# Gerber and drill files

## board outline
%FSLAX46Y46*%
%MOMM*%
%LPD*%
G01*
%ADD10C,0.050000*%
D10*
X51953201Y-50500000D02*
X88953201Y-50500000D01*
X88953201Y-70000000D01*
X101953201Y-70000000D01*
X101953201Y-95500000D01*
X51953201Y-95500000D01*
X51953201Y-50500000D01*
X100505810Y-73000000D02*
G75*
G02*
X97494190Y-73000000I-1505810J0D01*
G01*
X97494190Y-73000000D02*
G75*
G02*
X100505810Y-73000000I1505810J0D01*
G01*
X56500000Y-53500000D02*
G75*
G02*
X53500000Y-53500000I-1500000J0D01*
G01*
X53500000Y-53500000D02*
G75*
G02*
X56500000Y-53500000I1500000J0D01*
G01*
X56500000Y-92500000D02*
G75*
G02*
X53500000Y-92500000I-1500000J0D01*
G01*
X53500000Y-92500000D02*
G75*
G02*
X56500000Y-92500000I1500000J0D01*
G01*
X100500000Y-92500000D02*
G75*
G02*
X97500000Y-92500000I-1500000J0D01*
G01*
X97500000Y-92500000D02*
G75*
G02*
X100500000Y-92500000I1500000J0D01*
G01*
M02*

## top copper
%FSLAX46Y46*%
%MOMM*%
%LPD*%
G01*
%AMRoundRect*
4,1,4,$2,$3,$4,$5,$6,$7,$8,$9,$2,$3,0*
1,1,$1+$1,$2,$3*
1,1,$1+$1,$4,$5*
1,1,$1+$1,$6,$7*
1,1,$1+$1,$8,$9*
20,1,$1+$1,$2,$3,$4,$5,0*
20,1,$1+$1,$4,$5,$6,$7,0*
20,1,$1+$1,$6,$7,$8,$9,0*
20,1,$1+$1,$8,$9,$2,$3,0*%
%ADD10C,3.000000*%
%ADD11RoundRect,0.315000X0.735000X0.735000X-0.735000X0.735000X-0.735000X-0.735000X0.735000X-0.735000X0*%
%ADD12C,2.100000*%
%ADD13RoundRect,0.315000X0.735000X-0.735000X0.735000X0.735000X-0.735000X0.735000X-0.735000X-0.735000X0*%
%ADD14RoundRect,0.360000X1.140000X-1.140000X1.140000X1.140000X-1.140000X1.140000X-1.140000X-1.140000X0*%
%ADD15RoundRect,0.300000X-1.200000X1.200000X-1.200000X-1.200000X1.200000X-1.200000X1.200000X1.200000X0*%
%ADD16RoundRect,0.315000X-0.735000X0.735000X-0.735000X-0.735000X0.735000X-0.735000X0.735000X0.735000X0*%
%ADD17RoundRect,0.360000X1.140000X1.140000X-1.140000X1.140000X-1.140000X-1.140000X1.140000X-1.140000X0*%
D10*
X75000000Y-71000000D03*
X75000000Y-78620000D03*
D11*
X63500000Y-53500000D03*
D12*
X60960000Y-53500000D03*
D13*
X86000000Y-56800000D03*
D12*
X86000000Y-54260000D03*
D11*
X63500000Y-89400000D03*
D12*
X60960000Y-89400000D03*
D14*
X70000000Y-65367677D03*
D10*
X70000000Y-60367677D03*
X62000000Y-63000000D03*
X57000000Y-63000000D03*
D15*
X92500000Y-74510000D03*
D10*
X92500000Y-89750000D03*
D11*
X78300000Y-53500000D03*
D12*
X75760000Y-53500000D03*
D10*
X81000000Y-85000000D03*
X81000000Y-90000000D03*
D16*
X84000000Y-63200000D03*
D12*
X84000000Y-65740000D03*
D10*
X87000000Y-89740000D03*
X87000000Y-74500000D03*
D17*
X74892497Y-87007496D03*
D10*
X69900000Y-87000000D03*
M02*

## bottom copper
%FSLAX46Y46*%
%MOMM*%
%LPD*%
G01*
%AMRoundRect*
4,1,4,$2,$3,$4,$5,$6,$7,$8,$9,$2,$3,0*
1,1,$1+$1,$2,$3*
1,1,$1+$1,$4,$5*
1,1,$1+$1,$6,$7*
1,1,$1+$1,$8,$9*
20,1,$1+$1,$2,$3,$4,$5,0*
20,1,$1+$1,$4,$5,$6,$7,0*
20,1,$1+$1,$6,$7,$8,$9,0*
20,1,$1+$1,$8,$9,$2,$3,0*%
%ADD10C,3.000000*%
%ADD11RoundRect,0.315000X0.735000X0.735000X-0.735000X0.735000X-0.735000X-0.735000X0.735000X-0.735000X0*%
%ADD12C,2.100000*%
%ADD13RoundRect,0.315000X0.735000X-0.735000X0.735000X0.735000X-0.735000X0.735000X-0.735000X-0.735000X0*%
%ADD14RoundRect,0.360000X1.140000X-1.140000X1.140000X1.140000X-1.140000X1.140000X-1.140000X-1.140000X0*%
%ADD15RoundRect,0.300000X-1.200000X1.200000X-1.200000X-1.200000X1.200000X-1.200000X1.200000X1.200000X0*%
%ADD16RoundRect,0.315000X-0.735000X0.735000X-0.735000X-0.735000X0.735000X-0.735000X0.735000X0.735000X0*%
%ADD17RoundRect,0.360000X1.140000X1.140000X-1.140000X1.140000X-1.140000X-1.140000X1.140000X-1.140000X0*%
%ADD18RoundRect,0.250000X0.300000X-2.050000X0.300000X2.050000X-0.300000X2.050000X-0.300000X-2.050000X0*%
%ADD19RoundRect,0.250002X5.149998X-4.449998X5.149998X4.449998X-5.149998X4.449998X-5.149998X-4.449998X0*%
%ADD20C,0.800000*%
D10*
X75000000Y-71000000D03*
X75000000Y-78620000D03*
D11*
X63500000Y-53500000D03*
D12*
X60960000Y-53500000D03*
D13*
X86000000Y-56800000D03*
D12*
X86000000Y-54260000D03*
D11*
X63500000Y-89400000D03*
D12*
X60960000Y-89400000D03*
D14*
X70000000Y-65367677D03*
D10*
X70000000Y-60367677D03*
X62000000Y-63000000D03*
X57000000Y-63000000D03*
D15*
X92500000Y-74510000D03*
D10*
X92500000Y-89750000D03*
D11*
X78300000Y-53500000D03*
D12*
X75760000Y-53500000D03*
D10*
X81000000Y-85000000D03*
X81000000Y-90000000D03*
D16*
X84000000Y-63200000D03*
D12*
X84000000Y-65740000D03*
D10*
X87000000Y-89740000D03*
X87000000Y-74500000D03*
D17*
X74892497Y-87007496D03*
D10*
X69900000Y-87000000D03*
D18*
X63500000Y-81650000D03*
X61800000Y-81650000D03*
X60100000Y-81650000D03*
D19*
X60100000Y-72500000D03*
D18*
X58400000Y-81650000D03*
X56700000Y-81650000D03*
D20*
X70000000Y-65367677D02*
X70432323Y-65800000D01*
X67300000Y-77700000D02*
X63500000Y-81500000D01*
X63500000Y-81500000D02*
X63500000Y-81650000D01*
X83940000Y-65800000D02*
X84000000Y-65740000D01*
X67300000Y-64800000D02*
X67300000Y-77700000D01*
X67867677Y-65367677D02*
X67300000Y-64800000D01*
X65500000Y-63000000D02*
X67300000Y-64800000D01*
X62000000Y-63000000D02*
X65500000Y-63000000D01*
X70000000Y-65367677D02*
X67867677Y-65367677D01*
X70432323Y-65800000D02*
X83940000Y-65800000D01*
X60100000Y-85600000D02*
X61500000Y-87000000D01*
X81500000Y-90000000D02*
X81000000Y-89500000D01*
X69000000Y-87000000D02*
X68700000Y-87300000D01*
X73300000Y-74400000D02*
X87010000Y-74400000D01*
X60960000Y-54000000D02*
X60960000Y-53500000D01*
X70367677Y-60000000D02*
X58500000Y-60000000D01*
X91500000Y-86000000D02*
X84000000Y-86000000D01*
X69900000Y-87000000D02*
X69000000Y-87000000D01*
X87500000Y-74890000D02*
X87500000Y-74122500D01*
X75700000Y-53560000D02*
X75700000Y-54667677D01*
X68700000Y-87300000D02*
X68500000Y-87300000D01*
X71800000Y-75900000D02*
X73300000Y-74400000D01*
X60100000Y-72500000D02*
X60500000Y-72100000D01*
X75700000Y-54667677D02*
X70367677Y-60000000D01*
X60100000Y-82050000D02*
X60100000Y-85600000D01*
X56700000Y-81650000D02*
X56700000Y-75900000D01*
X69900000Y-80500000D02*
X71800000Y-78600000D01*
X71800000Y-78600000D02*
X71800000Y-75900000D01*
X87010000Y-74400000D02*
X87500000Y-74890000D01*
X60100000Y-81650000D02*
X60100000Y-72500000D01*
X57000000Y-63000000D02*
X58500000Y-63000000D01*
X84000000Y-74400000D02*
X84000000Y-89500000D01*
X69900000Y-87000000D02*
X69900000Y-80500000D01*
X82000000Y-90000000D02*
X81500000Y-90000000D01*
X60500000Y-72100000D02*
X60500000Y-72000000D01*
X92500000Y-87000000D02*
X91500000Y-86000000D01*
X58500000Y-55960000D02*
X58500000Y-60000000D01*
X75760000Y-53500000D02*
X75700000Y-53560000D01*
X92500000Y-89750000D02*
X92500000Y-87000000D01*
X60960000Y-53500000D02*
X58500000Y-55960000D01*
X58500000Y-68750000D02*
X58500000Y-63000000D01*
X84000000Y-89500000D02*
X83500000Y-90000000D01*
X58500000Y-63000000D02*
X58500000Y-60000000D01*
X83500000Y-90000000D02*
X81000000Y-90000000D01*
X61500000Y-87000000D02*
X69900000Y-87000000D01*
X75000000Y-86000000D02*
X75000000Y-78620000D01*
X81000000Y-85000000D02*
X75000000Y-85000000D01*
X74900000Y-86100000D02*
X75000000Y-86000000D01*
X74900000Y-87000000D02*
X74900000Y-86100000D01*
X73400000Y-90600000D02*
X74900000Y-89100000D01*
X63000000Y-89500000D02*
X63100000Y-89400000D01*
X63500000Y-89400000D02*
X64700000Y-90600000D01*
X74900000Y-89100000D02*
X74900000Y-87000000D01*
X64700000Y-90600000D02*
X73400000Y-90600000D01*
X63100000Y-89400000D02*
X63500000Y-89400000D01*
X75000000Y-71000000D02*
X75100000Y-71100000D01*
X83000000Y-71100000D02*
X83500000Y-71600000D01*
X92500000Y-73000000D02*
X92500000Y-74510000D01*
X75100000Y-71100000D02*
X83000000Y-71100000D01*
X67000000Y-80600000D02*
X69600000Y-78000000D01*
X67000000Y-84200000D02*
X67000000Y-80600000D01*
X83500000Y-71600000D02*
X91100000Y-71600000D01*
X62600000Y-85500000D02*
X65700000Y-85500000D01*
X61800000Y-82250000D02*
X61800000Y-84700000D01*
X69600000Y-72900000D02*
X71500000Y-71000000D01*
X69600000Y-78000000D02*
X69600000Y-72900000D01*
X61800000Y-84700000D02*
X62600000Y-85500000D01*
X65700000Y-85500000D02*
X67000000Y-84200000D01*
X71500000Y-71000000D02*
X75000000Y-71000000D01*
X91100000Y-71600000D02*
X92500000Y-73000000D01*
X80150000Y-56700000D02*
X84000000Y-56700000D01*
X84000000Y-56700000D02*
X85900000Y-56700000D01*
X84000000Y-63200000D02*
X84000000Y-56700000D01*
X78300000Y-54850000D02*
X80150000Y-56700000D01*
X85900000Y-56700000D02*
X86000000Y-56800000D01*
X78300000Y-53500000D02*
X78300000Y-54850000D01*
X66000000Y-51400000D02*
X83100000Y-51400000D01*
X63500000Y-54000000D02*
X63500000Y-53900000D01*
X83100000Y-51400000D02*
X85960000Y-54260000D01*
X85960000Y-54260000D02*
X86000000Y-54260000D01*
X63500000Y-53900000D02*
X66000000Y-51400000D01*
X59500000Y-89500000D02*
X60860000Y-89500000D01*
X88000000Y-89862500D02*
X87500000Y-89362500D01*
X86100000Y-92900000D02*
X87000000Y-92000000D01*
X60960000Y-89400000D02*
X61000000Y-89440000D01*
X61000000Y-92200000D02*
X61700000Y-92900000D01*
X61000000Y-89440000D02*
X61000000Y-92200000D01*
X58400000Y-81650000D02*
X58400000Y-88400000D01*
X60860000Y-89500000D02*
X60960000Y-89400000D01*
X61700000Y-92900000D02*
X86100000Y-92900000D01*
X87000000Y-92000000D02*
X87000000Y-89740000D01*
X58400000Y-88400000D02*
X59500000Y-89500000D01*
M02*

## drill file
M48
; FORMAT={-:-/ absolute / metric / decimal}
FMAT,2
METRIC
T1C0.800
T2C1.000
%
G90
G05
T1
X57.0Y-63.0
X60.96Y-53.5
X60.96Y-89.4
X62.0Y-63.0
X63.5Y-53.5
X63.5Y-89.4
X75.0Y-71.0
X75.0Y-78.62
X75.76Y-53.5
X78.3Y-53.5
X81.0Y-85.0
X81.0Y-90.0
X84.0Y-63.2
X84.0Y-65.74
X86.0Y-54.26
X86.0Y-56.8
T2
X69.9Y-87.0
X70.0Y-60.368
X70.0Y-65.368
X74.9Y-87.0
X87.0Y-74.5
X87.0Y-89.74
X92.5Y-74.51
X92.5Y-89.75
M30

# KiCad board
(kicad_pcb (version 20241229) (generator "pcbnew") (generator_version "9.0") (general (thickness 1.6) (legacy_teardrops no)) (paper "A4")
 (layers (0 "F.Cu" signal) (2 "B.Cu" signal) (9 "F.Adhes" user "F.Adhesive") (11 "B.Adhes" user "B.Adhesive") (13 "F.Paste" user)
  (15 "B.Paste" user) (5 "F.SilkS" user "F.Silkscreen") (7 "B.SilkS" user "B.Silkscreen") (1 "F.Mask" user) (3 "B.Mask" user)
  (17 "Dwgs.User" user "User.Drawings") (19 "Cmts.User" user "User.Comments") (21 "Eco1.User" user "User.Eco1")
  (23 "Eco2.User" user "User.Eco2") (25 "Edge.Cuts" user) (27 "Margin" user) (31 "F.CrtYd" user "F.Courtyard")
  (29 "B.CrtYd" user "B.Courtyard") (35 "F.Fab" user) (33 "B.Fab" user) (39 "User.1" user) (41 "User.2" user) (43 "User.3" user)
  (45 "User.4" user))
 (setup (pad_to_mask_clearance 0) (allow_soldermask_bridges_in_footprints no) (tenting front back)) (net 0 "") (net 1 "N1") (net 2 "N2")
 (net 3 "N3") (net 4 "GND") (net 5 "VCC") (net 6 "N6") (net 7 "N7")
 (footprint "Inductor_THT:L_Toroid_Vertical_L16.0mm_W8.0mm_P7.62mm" (layer "F.Cu") (at 75 71)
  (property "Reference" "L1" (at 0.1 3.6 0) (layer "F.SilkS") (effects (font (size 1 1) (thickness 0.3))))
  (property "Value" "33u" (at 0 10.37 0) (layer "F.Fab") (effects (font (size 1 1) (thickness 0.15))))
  (pad "1" thru_hole circle (at 0 0) (size 3 3) (drill 0.8) (layers "*.Cu" "*.Mask") (remove_unused_layers no) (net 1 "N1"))
  (pad "2" thru_hole circle (at 0 7.62) (size 3 3) (drill 0.8) (layers "*.Cu" "*.Mask") (remove_unused_layers no) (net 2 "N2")))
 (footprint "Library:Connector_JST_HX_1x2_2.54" (layer "F.Cu") (at 63.5 53.5 180)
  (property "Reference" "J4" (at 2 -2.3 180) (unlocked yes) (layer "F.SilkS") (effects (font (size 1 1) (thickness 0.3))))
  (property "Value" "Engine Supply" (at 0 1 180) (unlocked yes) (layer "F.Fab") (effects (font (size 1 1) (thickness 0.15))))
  (pad "1" thru_hole roundrect (at 0 0 180) (size 2.1 2.1) (drill 0.8) (layers "*.Cu" "*.Mask") (remove_unused_layers no)
   (roundrect_rratio 0.15) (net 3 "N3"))
  (pad "2" thru_hole circle (at 2.54 0 180) (size 2.1 2.1) (drill 0.8) (layers "*.Cu" "*.Mask") (remove_unused_layers no) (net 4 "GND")))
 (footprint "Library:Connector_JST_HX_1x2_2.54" (layer "F.Cu") (at 86 56.8 90)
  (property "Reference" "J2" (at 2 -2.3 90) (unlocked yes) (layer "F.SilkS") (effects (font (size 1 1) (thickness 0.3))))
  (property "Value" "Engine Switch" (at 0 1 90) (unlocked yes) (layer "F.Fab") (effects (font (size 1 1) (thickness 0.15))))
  (pad "1" thru_hole roundrect (at 0 0 90) (size 2.1 2.1) (drill 0.8) (layers "*.Cu" "*.Mask") (remove_unused_layers no)
   (roundrect_rratio 0.15) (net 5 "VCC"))
  (pad "2" thru_hole circle (at 2.54 0 90) (size 2.1 2.1) (drill 0.8) (layers "*.Cu" "*.Mask") (remove_unused_layers no) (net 3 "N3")))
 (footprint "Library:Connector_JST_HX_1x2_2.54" (layer "F.Cu") (at 63.5 89.4 180)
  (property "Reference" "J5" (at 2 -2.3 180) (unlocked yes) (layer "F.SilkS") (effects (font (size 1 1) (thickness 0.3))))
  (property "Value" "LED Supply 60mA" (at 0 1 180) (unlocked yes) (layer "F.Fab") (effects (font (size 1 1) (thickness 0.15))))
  (pad "1" thru_hole roundrect (at 0 0 180) (size 2.1 2.1) (drill 0.8) (layers "*.Cu" "*.Mask") (remove_unused_layers no)
   (roundrect_rratio 0.15) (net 2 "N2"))
  (pad "2" thru_hole circle (at 2.54 0 180) (size 2.1 2.1) (drill 0.8) (layers "*.Cu" "*.Mask") (remove_unused_layers no) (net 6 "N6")))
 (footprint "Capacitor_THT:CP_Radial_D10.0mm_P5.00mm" (layer "F.Cu") (at 70 65.367677 90)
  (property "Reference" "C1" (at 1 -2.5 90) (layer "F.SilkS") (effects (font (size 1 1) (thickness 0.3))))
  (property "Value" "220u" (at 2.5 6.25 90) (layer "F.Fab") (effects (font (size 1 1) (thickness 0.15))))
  (pad "1" thru_hole roundrect (at 0 0 90) (size 3 3) (drill 1) (layers "*.Cu" "*.Mask") (remove_unused_layers no) (roundrect_rratio 0.12)
   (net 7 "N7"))
  (pad "2" thru_hole circle (at 5 0 90) (size 3 3) (drill 1) (layers "*.Cu" "*.Mask") (remove_unused_layers no) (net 4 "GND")))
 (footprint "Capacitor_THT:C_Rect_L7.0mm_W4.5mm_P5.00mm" (layer "F.Cu") (at 62 63 180)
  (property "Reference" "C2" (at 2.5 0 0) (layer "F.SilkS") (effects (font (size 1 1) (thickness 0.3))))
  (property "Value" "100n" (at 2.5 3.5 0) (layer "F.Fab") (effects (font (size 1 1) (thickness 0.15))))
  (pad "1" thru_hole circle (at 0 0 180) (size 3 3) (drill 0.8) (layers "*.Cu" "*.Mask") (remove_unused_layers no) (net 7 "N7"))
  (pad "2" thru_hole circle (at 5 0 180) (size 3 3) (drill 0.8) (layers "*.Cu" "*.Mask") (remove_unused_layers no) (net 4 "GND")))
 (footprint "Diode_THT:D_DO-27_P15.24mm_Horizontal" (layer "F.Cu") (at 92.5 74.51 -90)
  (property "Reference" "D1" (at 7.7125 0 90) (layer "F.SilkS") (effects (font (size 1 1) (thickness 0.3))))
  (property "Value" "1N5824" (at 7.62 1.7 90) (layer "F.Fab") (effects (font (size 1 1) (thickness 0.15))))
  (pad "1" thru_hole roundrect (at 0 0 270) (size 3 3) (drill 1) (layers "*.Cu" "*.Mask") (remove_unused_layers no) (roundrect_rratio 0.1)
   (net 1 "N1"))
  (pad "2" thru_hole circle (at 15.24 0 270) (size 3 3) (drill 1) (layers "*.Cu" "*.Mask") (remove_unused_layers no) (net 4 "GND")))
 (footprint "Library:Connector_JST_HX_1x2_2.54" (layer "F.Cu") (at 78.3 53.5 180)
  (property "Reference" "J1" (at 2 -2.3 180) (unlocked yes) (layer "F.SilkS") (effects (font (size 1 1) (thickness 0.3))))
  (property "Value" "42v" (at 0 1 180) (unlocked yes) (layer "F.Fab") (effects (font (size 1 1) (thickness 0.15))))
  (pad "1" thru_hole roundrect (at 0 0 180) (size 2.1 2.1) (drill 0.8) (layers "*.Cu" "*.Mask") (remove_unused_layers no)
   (roundrect_rratio 0.15) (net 5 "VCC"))
  (pad "2" thru_hole circle (at 2.54 0 180) (size 2.1 2.1) (drill 0.8) (layers "*.Cu" "*.Mask") (remove_unused_layers no) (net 4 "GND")))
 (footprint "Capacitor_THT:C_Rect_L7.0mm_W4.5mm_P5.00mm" (layer "F.Cu") (at 81 85 -90)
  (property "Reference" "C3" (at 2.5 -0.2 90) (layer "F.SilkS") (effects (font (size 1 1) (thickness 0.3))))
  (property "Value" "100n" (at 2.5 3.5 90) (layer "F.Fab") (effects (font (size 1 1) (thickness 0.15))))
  (pad "1" thru_hole circle (at 0 0 270) (size 3 3) (drill 0.8) (layers "*.Cu" "*.Mask") (remove_unused_layers no) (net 2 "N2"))
  (pad "2" thru_hole circle (at 5 0 270) (size 3 3) (drill 0.8) (layers "*.Cu" "*.Mask") (remove_unused_layers no) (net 4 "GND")))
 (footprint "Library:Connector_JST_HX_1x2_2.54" (layer "F.Cu") (at 84 63.2 -90)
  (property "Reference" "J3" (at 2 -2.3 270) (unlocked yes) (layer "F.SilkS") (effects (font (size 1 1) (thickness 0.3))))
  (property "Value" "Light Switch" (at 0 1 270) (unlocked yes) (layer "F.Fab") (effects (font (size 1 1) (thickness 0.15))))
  (pad "1" thru_hole roundrect (at 0 0 270) (size 2.1 2.1) (drill 0.8) (layers "*.Cu" "*.Mask") (remove_unused_layers no)
   (roundrect_rratio 0.15) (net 5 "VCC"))
  (pad "2" thru_hole circle (at 2.54 0 270) (size 2.1 2.1) (drill 0.8) (layers "*.Cu" "*.Mask") (remove_unused_layers no) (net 7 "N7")))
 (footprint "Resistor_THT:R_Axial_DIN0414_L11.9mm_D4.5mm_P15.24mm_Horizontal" (layer "F.Cu") (at 87 89.74 90)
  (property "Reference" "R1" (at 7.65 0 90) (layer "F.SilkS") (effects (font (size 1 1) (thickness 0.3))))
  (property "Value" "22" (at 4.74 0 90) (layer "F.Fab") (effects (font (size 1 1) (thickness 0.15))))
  (pad "1" thru_hole circle (at 0 0 90) (size 3 3) (drill 1) (layers "*.Cu" "*.Mask") (remove_unused_layers no) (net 6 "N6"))
  (pad "2" thru_hole circle (at 15.24 0 90) (size 3 3) (drill 1) (layers "*.Cu" "*.Mask") (remove_unused_layers no) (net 4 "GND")))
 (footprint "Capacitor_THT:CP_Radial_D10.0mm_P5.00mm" (layer "F.Cu") (at 74.9 87 180)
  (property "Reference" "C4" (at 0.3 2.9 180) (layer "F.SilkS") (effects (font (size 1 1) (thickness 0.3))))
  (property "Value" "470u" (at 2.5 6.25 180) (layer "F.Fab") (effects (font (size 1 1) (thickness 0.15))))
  (pad "1" thru_hole roundrect (at 0 0 180) (size 3 3) (drill 1 (offset 0.007503 -0.007496)) (layers "*.Cu" "*.Mask")
   (remove_unused_layers no) (roundrect_rratio 0.12) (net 2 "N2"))
  (pad "2" thru_hole circle (at 5 0 180) (size 3 3) (drill 1) (layers "*.Cu" "*.Mask") (remove_unused_layers no) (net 4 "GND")))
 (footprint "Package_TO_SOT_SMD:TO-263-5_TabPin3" (layer "B.Cu") (at 60.1 74 90)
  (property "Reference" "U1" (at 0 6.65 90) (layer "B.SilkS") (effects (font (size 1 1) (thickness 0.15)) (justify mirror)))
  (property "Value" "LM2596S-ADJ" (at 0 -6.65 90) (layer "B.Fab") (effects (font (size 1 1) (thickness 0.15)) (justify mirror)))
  (pad "" smd roundrect (at -0.925 -2.775 90) (size 4.55 5.25) (layers "B.Paste") (roundrect_rratio 0.054945))
  (pad "" smd roundrect (at -0.925 2.775 90) (size 4.55 5.25) (layers "B.Paste") (roundrect_rratio 0.054945))
  (pad "" smd roundrect (at 3.925 -2.775 90) (size 4.55 5.25) (layers "B.Paste") (roundrect_rratio 0.054945))
  (pad "" smd roundrect (at 3.925 2.775 90) (size 4.55 5.25) (layers "B.Paste") (roundrect_rratio 0.054945))
  (pad "1" smd roundrect (at -7.65 3.4 90) (size 4.6 1.1) (layers "B.Cu" "B.Mask" "B.Paste") (roundrect_rratio 0.227273) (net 7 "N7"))
  (pad "2" smd roundrect (at -7.65 1.7 90) (size 4.6 1.1) (layers "B.Cu" "B.Mask" "B.Paste") (roundrect_rratio 0.227273) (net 1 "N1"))
  (pad "3" smd roundrect (at -7.65 0 90) (size 4.6 1.1) (layers "B.Cu" "B.Mask" "B.Paste") (roundrect_rratio 0.227273) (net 4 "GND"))
  (pad "3" smd roundrect (at 1.5 0 90) (size 9.4 10.8) (layers "B.Cu" "B.Mask") (roundrect_rratio 0.026596) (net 4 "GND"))
  (pad "4" smd roundrect (at -7.65 -1.7 90) (size 4.6 1.1) (layers "B.Cu" "B.Mask" "B.Paste") (roundrect_rratio 0.227273) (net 6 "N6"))
  (pad "5" smd roundrect (at -7.65 -3.4 90) (size 4.6 1.1) (layers "B.Cu" "B.Mask" "B.Paste") (roundrect_rratio 0.227273) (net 4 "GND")))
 (gr_poly
  (pts (xy 51.953201 50.5) (xy 88.953201 50.5) (xy 88.953201 70) (xy 101.953201 70) (xy 101.953201 95.5) (xy 51.953201 95.5))
  (stroke (width 0.05) (type solid)) (fill no) (layer "Edge.Cuts"))
 (gr_circle (center 99 73) (end 99 71.49419) (stroke (width 0.05) (type default)) (fill no) (layer "Edge.Cuts"))
 (gr_circle (center 55 53.5) (end 55 52) (stroke (width 0.05) (type default)) (fill no) (layer "Edge.Cuts"))
 (gr_circle (center 55 92.5) (end 55 91) (stroke (width 0.05) (type default)) (fill no) (layer "Edge.Cuts"))
 (gr_circle (center 99 92.5) (end 99 94) (stroke (width 0.05) (type default)) (fill no) (layer "Edge.Cuts"))
 (segment (start 70 65.367677) (end 70.432323 65.8) (width 0.8) (layer "B.Cu") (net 7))
 (segment (start 67.3 77.7) (end 63.5 81.5) (width 0.8) (layer "B.Cu") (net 7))
 (segment (start 63.5 81.5) (end 63.5 81.65) (width 0.8) (layer "B.Cu") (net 7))
 (segment (start 83.94 65.8) (end 84 65.74) (width 0.8) (layer "B.Cu") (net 7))
 (segment (start 67.3 64.8) (end 67.3 77.7) (width 0.8) (layer "B.Cu") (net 7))
 (segment (start 67.867677 65.367677) (end 67.3 64.8) (width 0.8) (layer "B.Cu") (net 7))
 (segment (start 65.5 63) (end 67.3 64.8) (width 0.8) (layer "B.Cu") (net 7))
 (segment (start 62 63) (end 65.5 63) (width 0.8) (layer "B.Cu") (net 7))
 (segment (start 70 65.367677) (end 67.867677 65.367677) (width 0.8) (layer "B.Cu") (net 7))
 (segment (start 70.432323 65.8) (end 83.94 65.8) (width 0.8) (layer "B.Cu") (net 7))
 (segment (start 60.1 85.6) (end 61.5 87) (width 0.8) (layer "B.Cu") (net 4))
 (segment (start 81.5 90) (end 81 89.5) (width 0.8) (layer "B.Cu") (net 4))
 (segment (start 69 87) (end 68.7 87.3) (width 0.8) (layer "B.Cu") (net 4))
 (segment (start 73.3 74.4) (end 87.01 74.4) (width 0.8) (layer "B.Cu") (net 4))
 (segment (start 60.96 54) (end 60.96 53.5) (width 0.8) (layer "B.Cu") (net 4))
 (segment (start 70.367677 60) (end 58.5 60) (width 0.8) (layer "B.Cu") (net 4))
 (segment (start 91.5 86) (end 84 86) (width 0.8) (layer "B.Cu") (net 4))
 (segment (start 69.9 87) (end 69 87) (width 0.8) (layer "B.Cu") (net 4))
 (segment (start 87.5 74.89) (end 87.5 74.1225) (width 0.8) (layer "B.Cu") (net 4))
 (segment (start 75.7 53.56) (end 75.7 54.667677) (width 0.8) (layer "B.Cu") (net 4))
 (segment (start 68.7 87.3) (end 68.5 87.3) (width 0.8) (layer "B.Cu") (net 4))
 (segment (start 71.8 75.9) (end 73.3 74.4) (width 0.8) (layer "B.Cu") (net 4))
 (segment (start 60.1 72.5) (end 60.5 72.1) (width 0.8) (layer "B.Cu") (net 4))
 (segment (start 75.7 54.667677) (end 70.367677 60) (width 0.8) (layer "B.Cu") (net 4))
 (segment (start 60.1 82.05) (end 60.1 85.6) (width 0.8) (layer "B.Cu") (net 4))
 (segment (start 56.7 81.65) (end 56.7 75.9) (width 0.8) (layer "B.Cu") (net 4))
 (segment (start 69.9 80.5) (end 71.8 78.6) (width 0.8) (layer "B.Cu") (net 4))
 (segment (start 71.8 78.6) (end 71.8 75.9) (width 0.8) (layer "B.Cu") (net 4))
 (segment (start 87.01 74.4) (end 87.5 74.89) (width 0.8) (layer "B.Cu") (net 4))
 (segment (start 60.1 81.65) (end 60.1 72.5) (width 0.8) (layer "B.Cu") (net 4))
 (segment (start 57 63) (end 58.5 63) (width 0.8) (layer "B.Cu") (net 4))
 (segment (start 84 74.4) (end 84 89.5) (width 0.8) (layer "B.Cu") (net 4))
 (segment (start 69.9 87) (end 69.9 80.5) (width 0.8) (layer "B.Cu") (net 4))
 (segment (start 82 90) (end 81.5 90) (width 0.8) (layer "B.Cu") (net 4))
 (segment (start 60.5 72.1) (end 60.5 72) (width 0.8) (layer "B.Cu") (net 4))
 (segment (start 92.5 87) (end 91.5 86) (width 0.8) (layer "B.Cu") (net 4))
 (segment (start 58.5 55.96) (end 58.5 60) (width 0.8) (layer "B.Cu") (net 4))
 (segment (start 75.76 53.5) (end 75.7 53.56) (width 0.8) (layer "B.Cu") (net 4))
 (segment (start 92.5 89.75) (end 92.5 87) (width 0.8) (layer "B.Cu") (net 4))
 (segment (start 60.96 53.5) (end 58.5 55.96) (width 0.8) (layer "B.Cu") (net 4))
 (segment (start 58.5 68.75) (end 58.5 63) (width 0.8) (layer "B.Cu") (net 4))
 (segment (start 84 89.5) (end 83.5 90) (width 0.8) (layer "B.Cu") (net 4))
 (segment (start 58.5 63) (end 58.5 60) (width 0.8) (layer "B.Cu") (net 4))
 (segment (start 83.5 90) (end 81 90) (width 0.8) (layer "B.Cu") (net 4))
 (segment (start 61.5 87) (end 69.9 87) (width 0.8) (layer "B.Cu") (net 4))
 (segment (start 75 86) (end 75 78.62) (width 0.8) (layer "B.Cu") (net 2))
 (segment (start 81 85) (end 75 85) (width 0.8) (layer "B.Cu") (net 2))
 (segment (start 74.9 86.1) (end 75 86) (width 0.8) (layer "B.Cu") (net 2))
 (segment (start 74.9 87) (end 74.9 86.1) (width 0.8) (layer "B.Cu") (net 2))
 (segment (start 73.4 90.6) (end 74.9 89.1) (width 0.8) (layer "B.Cu") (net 2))
 (segment (start 63 89.5) (end 63.1 89.4) (width 0.8) (layer "B.Cu") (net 2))
 (segment (start 63.5 89.4) (end 64.7 90.6) (width 0.8) (layer "B.Cu") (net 2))
 (segment (start 74.9 89.1) (end 74.9 87) (width 0.8) (layer "B.Cu") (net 2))
 (segment (start 64.7 90.6) (end 73.4 90.6) (width 0.8) (layer "B.Cu") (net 2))
 (segment (start 63.1 89.4) (end 63.5 89.4) (width 0.8) (layer "B.Cu") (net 2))
 (segment (start 75 71) (end 75.1 71.1) (width 0.8) (layer "B.Cu") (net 1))
 (segment (start 83 71.1) (end 83.5 71.6) (width 0.8) (layer "B.Cu") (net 1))
 (segment (start 92.5 73) (end 92.5 74.51) (width 0.8) (layer "B.Cu") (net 1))
 (segment (start 75.1 71.1) (end 83 71.1) (width 0.8) (layer "B.Cu") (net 1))
 (segment (start 67 80.6) (end 69.6 78) (width 0.8) (layer "B.Cu") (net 1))
 (segment (start 67 84.2) (end 67 80.6) (width 0.8) (layer "B.Cu") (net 1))
 (segment (start 83.5 71.6) (end 91.1 71.6) (width 0.8) (layer "B.Cu") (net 1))
 (segment (start 62.6 85.5) (end 65.7 85.5) (width 0.8) (layer "B.Cu") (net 1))
 (segment (start 61.8 82.25) (end 61.8 84.7) (width 0.8) (layer "B.Cu") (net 1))
 (segment (start 69.6 72.9) (end 71.5 71) (width 0.8) (layer "B.Cu") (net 1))
 (segment (start 69.6 78) (end 69.6 72.9) (width 0.8) (layer "B.Cu") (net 1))
 (segment (start 61.8 84.7) (end 62.6 85.5) (width 0.8) (layer "B.Cu") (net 1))
 (segment (start 65.7 85.5) (end 67 84.2) (width 0.8) (layer "B.Cu") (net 1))
 (segment (start 71.5 71) (end 75 71) (width 0.8) (layer "B.Cu") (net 1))
 (segment (start 91.1 71.6) (end 92.5 73) (width 0.8) (layer "B.Cu") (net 1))
 (segment (start 80.15 56.7) (end 84 56.7) (width 0.8) (layer "B.Cu") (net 5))
 (segment (start 84 56.7) (end 85.9 56.7) (width 0.8) (layer "B.Cu") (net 5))
 (segment (start 84 63.2) (end 84 56.7) (width 0.8) (layer "B.Cu") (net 5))
 (segment (start 78.3 54.85) (end 80.15 56.7) (width 0.8) (layer "B.Cu") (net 5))
 (segment (start 85.9 56.7) (end 86 56.8) (width 0.8) (layer "B.Cu") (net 5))
 (segment (start 78.3 53.5) (end 78.3 54.85) (width 0.8) (layer "B.Cu") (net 5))
 (segment (start 66 51.4) (end 83.1 51.4) (width 0.8) (layer "B.Cu") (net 3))
 (segment (start 63.5 54) (end 63.5 53.9) (width 0.8) (layer "B.Cu") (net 3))
 (segment (start 83.1 51.4) (end 85.96 54.26) (width 0.8) (layer "B.Cu") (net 3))
 (segment (start 85.96 54.26) (end 86 54.26) (width 0.8) (layer "B.Cu") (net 3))
 (segment (start 63.5 53.9) (end 66 51.4) (width 0.8) (layer "B.Cu") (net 3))
 (segment (start 59.5 89.5) (end 60.86 89.5) (width 0.8) (layer "B.Cu") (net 6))
 (segment (start 88 89.8625) (end 87.5 89.3625) (width 0.8) (layer "B.Cu") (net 6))
 (segment (start 86.1 92.9) (end 87 92) (width 0.8) (layer "B.Cu") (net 6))
 (segment (start 60.96 89.4) (end 61 89.44) (width 0.8) (layer "B.Cu") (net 6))
 (segment (start 61 92.2) (end 61.7 92.9) (width 0.8) (layer "B.Cu") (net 6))
 (segment (start 61 89.44) (end 61 92.2) (width 0.8) (layer "B.Cu") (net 6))
 (segment (start 58.4 81.65) (end 58.4 88.4) (width 0.8) (layer "B.Cu") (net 6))
 (segment (start 60.86 89.5) (end 60.96 89.4) (width 0.8) (layer "B.Cu") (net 6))
 (segment (start 61.7 92.9) (end 86.1 92.9) (width 0.8) (layer "B.Cu") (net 6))
 (segment (start 87 92) (end 87 89.74) (width 0.8) (layer "B.Cu") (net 6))
 (segment (start 58.4 88.4) (end 59.5 89.5) (width 0.8) (layer "B.Cu") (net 6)))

